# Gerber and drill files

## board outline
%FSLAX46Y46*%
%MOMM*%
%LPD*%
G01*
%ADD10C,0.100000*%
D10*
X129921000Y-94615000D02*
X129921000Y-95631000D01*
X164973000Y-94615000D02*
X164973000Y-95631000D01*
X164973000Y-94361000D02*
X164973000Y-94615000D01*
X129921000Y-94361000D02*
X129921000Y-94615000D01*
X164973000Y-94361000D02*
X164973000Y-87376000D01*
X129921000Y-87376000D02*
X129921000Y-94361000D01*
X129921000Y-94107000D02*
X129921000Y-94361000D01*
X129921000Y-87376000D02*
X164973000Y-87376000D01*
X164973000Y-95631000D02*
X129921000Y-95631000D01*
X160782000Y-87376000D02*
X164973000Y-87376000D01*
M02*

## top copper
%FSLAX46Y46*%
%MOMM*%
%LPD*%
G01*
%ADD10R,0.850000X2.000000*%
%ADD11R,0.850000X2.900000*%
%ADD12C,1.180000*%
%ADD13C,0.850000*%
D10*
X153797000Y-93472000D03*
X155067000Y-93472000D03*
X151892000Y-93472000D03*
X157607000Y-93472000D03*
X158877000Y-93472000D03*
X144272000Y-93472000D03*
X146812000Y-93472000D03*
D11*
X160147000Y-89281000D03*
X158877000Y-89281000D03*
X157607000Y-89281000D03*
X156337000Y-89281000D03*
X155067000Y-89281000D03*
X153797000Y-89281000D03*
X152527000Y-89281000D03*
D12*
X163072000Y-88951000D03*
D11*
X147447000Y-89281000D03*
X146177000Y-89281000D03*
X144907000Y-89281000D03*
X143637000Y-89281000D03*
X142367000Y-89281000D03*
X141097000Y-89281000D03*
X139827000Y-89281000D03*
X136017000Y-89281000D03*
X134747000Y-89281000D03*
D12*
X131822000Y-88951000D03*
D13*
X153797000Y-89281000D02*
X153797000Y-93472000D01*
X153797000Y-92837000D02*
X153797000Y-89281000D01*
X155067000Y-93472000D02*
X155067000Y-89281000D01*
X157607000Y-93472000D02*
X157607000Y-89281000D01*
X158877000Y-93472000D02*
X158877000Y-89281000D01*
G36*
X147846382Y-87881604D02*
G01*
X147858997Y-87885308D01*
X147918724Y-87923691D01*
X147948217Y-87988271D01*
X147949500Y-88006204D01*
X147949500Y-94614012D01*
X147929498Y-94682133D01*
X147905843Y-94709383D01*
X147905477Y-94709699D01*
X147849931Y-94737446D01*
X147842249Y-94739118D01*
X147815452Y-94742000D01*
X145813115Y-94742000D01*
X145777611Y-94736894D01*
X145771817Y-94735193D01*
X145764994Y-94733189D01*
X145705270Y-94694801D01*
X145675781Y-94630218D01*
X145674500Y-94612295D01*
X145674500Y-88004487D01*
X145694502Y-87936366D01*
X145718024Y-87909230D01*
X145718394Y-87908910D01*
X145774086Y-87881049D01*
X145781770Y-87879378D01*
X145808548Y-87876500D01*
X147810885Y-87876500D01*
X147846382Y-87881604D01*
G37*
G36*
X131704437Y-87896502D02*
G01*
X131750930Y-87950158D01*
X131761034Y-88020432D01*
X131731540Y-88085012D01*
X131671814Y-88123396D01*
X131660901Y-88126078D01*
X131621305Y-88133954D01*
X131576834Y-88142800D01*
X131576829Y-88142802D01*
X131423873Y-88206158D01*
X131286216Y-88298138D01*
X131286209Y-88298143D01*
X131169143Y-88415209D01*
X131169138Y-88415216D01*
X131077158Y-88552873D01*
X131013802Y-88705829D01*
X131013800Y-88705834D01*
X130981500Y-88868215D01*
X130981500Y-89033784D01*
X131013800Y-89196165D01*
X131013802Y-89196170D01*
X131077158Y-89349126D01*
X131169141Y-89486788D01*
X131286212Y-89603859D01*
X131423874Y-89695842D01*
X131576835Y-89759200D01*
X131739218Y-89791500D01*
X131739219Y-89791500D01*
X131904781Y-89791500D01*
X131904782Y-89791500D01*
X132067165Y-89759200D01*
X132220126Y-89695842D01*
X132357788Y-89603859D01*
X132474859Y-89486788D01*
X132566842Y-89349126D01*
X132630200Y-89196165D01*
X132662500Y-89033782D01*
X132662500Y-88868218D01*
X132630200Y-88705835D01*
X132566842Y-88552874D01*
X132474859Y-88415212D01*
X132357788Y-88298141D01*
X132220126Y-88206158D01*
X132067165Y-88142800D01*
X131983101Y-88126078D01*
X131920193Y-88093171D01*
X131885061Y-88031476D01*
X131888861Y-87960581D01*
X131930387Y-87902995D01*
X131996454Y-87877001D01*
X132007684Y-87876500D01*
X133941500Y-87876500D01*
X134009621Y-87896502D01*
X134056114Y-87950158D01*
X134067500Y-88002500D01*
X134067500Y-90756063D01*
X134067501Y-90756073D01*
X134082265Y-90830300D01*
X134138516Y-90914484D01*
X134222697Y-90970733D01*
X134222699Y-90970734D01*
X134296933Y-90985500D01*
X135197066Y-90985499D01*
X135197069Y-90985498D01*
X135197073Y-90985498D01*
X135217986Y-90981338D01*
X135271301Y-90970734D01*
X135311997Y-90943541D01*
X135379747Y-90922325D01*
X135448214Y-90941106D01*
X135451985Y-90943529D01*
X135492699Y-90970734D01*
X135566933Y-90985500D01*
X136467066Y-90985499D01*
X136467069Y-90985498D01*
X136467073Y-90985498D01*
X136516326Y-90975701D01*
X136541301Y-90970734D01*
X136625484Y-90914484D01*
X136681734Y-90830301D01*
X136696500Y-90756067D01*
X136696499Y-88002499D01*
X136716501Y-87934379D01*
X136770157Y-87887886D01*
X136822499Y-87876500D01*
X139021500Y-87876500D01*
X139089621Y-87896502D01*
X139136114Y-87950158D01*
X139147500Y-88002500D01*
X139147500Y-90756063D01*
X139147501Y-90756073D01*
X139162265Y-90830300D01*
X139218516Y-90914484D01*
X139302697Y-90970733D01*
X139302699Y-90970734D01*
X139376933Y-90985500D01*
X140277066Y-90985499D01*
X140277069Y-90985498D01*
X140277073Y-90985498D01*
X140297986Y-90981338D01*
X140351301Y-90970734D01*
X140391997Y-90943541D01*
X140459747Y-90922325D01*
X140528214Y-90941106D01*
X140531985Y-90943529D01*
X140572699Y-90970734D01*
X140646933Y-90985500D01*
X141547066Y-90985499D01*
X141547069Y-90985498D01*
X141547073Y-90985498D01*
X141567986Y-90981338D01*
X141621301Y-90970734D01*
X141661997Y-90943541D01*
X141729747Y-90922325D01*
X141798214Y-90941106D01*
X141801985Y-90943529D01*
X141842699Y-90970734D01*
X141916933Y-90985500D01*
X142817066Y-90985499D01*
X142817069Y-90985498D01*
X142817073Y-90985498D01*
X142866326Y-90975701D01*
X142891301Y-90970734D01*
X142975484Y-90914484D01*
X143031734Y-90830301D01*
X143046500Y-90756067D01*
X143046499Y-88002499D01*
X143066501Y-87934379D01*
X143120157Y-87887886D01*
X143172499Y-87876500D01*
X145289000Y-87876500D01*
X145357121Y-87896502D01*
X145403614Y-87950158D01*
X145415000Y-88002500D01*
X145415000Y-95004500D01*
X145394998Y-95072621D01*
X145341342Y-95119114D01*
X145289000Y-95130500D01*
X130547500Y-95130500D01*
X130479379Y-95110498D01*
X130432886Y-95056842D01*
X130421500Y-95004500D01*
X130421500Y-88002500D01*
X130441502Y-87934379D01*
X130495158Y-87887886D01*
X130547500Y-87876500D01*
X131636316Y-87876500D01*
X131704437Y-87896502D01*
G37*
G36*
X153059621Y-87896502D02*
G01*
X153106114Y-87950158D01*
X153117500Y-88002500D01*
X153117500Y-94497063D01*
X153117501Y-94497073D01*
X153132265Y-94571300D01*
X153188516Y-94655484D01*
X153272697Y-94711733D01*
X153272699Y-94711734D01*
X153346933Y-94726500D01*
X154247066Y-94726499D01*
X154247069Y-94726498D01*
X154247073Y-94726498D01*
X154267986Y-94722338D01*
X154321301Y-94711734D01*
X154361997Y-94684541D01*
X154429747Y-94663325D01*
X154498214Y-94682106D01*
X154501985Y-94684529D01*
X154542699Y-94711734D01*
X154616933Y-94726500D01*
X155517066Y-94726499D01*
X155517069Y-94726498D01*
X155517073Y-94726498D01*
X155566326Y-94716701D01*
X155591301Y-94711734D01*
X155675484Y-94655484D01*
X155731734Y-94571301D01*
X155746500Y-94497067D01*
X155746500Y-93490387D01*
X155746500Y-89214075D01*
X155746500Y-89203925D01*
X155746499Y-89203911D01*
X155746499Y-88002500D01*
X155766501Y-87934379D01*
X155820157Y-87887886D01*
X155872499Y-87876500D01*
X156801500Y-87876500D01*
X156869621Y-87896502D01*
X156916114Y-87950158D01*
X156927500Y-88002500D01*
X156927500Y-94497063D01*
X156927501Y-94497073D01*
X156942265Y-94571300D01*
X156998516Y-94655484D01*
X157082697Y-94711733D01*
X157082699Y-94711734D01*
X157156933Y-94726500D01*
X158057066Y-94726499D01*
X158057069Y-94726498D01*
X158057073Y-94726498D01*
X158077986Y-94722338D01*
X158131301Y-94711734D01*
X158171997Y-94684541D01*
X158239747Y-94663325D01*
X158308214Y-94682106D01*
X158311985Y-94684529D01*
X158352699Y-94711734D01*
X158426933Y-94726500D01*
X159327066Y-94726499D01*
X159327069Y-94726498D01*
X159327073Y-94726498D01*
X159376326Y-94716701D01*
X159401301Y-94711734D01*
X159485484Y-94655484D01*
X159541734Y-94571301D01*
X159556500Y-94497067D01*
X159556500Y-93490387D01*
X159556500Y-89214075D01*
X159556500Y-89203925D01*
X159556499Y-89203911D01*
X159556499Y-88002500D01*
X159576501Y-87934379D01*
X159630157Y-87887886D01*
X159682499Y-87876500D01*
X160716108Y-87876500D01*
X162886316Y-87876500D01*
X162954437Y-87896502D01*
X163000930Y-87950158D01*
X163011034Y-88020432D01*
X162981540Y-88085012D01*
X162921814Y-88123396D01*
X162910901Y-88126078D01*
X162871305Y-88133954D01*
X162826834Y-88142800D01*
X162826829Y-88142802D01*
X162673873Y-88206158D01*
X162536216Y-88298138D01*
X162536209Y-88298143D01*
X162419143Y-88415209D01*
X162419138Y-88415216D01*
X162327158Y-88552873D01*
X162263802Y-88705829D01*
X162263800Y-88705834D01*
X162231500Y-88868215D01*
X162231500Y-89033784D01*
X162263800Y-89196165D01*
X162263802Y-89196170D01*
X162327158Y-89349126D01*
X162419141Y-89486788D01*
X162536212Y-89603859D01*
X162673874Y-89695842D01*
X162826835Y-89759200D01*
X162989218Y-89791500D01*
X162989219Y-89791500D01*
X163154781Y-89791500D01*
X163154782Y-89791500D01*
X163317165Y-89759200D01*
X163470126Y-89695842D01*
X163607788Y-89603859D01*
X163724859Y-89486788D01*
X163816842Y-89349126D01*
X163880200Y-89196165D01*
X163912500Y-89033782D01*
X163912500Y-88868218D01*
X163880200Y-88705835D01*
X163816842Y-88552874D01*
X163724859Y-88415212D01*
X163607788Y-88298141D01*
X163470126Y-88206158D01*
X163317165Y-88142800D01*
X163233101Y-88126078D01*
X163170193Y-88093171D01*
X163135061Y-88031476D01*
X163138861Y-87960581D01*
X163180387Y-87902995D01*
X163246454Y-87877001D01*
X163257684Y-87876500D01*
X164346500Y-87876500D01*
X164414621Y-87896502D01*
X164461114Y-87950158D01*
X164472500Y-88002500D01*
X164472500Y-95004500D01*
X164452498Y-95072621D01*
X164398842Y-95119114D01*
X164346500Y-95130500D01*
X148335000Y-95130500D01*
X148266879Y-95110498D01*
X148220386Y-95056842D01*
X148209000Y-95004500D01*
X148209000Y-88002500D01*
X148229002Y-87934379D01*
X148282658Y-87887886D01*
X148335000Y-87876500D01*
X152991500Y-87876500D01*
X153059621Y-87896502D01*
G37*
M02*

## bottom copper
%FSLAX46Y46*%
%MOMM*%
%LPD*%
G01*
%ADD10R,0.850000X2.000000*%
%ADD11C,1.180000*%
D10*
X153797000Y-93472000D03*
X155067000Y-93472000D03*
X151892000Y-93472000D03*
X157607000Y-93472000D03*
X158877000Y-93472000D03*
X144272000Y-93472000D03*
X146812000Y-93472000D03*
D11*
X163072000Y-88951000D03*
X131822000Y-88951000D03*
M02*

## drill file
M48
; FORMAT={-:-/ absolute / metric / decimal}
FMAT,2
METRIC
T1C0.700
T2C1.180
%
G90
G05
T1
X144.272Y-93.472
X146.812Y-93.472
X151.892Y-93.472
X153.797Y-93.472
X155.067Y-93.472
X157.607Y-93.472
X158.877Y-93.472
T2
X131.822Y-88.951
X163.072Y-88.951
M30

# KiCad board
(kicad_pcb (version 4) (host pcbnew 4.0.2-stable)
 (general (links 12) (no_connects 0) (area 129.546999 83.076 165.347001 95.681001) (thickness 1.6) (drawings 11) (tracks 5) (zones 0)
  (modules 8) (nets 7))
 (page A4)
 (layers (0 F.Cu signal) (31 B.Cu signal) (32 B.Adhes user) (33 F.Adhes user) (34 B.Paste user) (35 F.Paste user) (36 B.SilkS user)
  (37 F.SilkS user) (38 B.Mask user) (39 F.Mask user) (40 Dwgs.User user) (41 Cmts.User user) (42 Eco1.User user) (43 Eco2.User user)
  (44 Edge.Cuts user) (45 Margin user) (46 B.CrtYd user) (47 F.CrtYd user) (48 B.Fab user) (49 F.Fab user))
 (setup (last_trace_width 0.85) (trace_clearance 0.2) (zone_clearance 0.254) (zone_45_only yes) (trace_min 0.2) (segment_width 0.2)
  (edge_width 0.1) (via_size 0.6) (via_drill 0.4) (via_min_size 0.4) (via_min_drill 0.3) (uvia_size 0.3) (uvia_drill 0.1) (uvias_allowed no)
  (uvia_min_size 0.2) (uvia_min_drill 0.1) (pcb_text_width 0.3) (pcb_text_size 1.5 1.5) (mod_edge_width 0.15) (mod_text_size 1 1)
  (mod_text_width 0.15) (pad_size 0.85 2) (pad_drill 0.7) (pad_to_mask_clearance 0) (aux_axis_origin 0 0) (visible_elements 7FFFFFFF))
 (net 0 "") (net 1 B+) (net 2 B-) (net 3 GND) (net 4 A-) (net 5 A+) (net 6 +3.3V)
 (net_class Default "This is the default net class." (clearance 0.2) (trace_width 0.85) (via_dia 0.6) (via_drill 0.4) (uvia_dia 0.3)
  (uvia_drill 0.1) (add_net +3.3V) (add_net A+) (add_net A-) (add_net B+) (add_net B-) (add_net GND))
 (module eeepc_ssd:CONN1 (layer F.Cu) (at 153.797 93.472)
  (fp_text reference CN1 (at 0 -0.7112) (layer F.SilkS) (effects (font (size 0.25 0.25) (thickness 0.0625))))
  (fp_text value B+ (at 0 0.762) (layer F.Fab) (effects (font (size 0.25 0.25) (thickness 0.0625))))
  (pad 1 thru_hole rect (at 0 0) (size 0.85 2) (drill 0.7) (layers *.Cu *.Mask F.SilkS) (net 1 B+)))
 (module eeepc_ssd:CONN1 (layer F.Cu) (at 155.067 93.472)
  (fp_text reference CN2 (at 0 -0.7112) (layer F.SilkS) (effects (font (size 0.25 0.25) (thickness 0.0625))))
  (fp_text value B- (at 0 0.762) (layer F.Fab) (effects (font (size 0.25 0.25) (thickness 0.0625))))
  (pad 1 thru_hole rect (at 0 0) (size 0.85 2) (drill 0.7) (layers *.Cu *.Mask F.SilkS) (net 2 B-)))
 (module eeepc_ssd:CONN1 (layer F.Cu) (at 151.892 93.472)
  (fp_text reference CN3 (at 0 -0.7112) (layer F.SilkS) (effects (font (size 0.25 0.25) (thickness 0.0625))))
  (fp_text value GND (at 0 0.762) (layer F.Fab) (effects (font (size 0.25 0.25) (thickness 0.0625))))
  (pad 1 thru_hole rect (at 0 0) (size 0.85 2) (drill 0.7) (layers *.Cu *.Mask F.SilkS) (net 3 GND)))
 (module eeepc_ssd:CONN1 (layer F.Cu) (at 157.607 93.472)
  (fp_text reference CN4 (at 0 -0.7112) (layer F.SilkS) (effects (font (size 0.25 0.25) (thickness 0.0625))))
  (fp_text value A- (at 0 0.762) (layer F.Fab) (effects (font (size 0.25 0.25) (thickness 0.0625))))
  (pad 1 thru_hole rect (at 0 0) (size 0.85 2) (drill 0.7) (layers *.Cu *.Mask F.SilkS) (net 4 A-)))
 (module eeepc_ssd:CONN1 (layer F.Cu) (at 158.877 93.472)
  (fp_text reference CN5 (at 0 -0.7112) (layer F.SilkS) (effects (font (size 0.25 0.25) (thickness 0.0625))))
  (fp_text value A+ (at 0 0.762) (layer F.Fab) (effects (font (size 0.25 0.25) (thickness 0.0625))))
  (pad 1 thru_hole rect (at 0 0) (size 0.85 2) (drill 0.7) (layers *.Cu *.Mask F.SilkS) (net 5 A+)))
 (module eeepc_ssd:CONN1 (layer F.Cu) (at 144.272 93.472)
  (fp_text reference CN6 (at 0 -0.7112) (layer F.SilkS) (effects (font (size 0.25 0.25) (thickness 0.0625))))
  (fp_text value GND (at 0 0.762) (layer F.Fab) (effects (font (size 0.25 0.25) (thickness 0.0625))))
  (pad 1 thru_hole rect (at 0 0) (size 0.85 2) (drill 0.7) (layers *.Cu *.Mask F.SilkS) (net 3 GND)))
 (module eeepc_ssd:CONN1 (layer F.Cu) (at 146.812 93.472)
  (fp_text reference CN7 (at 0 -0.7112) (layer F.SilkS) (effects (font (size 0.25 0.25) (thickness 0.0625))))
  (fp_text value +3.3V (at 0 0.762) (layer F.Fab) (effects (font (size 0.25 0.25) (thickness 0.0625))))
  (pad 1 thru_hole rect (at 0 0) (size 0.85 2) (drill 0.7) (layers *.Cu *.Mask F.SilkS) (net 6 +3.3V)))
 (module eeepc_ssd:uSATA (layer F.Cu) (at 160.147 89.281)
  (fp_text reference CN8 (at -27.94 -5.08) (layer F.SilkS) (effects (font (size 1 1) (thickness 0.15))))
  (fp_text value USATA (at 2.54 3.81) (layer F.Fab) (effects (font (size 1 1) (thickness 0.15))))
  (pad 1 smd rect (at 0 0) (size 0.85 2.9) (layers F.Cu F.Paste F.Mask) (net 3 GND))
  (pad 2 smd rect (at -1.27 0) (size 0.85 2.9) (layers F.Cu F.Paste F.Mask) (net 5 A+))
  (pad 3 smd rect (at -2.54 0) (size 0.85 2.9) (layers F.Cu F.Paste F.Mask) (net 4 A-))
  (pad 4 smd rect (at -3.81 0) (size 0.85 2.9) (layers F.Cu F.Paste F.Mask) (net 3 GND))
  (pad 5 smd rect (at -5.08 0) (size 0.85 2.9) (layers F.Cu F.Paste F.Mask) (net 2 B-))
  (pad 6 smd rect (at -6.35 0) (size 0.85 2.9) (layers F.Cu F.Paste F.Mask) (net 1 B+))
  (pad 7 smd rect (at -7.62 0) (size 0.85 2.9) (layers F.Cu F.Paste F.Mask) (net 3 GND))
  (pad "" thru_hole circle (at 2.925 -0.33) (size 1.18 1.18) (drill 1.18) (layers *.Mask F.Cu F.SilkS) (clearance 0.0001))
  (pad 8 smd rect (at -12.7 0) (size 0.85 2.9) (layers F.Cu F.Paste F.Mask) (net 6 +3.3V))
  (pad 9 smd rect (at -13.97 0) (size 0.85 2.9) (layers F.Cu F.Paste F.Mask) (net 6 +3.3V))
  (pad 10 smd rect (at -15.24 0) (size 0.85 2.9) (layers F.Cu F.Paste F.Mask) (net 3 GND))
  (pad 11 smd rect (at -16.51 0) (size 0.85 2.9) (layers F.Cu F.Paste F.Mask) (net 3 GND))
  (pad 12 smd rect (at -17.78 0) (size 0.85 2.9) (layers F.Cu F.Paste F.Mask))
  (pad 13 smd rect (at -19.05 0) (size 0.85 2.9) (layers F.Cu F.Paste F.Mask))
  (pad 14 smd rect (at -20.32 0) (size 0.85 2.9) (layers F.Cu F.Paste F.Mask))
  (pad 15 smd rect (at -24.13 0) (size 0.85 2.9) (layers F.Cu F.Paste F.Mask))
  (pad 16 smd rect (at -25.4 0) (size 0.85 2.9) (layers F.Cu F.Paste F.Mask))
  (pad "" thru_hole circle (at -28.325 -0.33) (size 1.18 1.18) (drill 1.18) (layers *.Mask F.Cu F.SilkS) (clearance 0.0001)))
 (gr_line (start 129.921 94.615) (end 129.921 95.631) (angle 90) (layer Edge.Cuts) (width 0.1))
 (gr_line (start 164.973 94.615) (end 164.973 95.631) (angle 90) (layer Edge.Cuts) (width 0.1))
 (gr_line (start 164.973 94.361) (end 164.973 94.615) (angle 90) (layer Edge.Cuts) (width 0.1))
 (gr_line (start 129.921 94.361) (end 129.921 94.615) (angle 90) (layer Edge.Cuts) (width 0.1))
 (gr_line (start 164.973 94.361) (end 164.973 87.376) (angle 90) (layer Edge.Cuts) (width 0.1))
 (gr_line (start 129.921 87.376) (end 129.921 94.361) (angle 90) (layer Edge.Cuts) (width 0.1))
 (gr_line (start 129.921 94.107) (end 129.921 94.361) (angle 90) (layer Edge.Cuts) (width 0.1))
 (gr_line (start 129.921 87.376) (end 164.973 87.376) (angle 90) (layer Edge.Cuts) (width 0.1))
 (gr_line (start 164.973 95.631) (end 129.921 95.631) (angle 90) (layer Edge.Cuts) (width 0.1))
 (gr_line (start 160.782 87.376) (end 164.973 87.376) (angle 90) (layer Edge.Cuts) (width 0.1))
 (segment (start 153.797 89.281) (end 153.797 93.472) (width 0.85) (layer F.Cu) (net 1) (status C00000))
 (segment (start 153.797 92.837) (end 153.797 89.281) (width 0.85) (layer F.Cu) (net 1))
 (segment (start 155.067 93.472) (end 155.067 89.281) (width 0.85) (layer F.Cu) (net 2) (status 10))
 (segment (start 157.607 93.472) (end 157.607 89.281) (width 0.85) (layer F.Cu) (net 4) (status 10))
 (segment (start 158.877 93.472) (end 158.877 89.281) (width 0.85) (layer F.Cu) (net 5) (status 10))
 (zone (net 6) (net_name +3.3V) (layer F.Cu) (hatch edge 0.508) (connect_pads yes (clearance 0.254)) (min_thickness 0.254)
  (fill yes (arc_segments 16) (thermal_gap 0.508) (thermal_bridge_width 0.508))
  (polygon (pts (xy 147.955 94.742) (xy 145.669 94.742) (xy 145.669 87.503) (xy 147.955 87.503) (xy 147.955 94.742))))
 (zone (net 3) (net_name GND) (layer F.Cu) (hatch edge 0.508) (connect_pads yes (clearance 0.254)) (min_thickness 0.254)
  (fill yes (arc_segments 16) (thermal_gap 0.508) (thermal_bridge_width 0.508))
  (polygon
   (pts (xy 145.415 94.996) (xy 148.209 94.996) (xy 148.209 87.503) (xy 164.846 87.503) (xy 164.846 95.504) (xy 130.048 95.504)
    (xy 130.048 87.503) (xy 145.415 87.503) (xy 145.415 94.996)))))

